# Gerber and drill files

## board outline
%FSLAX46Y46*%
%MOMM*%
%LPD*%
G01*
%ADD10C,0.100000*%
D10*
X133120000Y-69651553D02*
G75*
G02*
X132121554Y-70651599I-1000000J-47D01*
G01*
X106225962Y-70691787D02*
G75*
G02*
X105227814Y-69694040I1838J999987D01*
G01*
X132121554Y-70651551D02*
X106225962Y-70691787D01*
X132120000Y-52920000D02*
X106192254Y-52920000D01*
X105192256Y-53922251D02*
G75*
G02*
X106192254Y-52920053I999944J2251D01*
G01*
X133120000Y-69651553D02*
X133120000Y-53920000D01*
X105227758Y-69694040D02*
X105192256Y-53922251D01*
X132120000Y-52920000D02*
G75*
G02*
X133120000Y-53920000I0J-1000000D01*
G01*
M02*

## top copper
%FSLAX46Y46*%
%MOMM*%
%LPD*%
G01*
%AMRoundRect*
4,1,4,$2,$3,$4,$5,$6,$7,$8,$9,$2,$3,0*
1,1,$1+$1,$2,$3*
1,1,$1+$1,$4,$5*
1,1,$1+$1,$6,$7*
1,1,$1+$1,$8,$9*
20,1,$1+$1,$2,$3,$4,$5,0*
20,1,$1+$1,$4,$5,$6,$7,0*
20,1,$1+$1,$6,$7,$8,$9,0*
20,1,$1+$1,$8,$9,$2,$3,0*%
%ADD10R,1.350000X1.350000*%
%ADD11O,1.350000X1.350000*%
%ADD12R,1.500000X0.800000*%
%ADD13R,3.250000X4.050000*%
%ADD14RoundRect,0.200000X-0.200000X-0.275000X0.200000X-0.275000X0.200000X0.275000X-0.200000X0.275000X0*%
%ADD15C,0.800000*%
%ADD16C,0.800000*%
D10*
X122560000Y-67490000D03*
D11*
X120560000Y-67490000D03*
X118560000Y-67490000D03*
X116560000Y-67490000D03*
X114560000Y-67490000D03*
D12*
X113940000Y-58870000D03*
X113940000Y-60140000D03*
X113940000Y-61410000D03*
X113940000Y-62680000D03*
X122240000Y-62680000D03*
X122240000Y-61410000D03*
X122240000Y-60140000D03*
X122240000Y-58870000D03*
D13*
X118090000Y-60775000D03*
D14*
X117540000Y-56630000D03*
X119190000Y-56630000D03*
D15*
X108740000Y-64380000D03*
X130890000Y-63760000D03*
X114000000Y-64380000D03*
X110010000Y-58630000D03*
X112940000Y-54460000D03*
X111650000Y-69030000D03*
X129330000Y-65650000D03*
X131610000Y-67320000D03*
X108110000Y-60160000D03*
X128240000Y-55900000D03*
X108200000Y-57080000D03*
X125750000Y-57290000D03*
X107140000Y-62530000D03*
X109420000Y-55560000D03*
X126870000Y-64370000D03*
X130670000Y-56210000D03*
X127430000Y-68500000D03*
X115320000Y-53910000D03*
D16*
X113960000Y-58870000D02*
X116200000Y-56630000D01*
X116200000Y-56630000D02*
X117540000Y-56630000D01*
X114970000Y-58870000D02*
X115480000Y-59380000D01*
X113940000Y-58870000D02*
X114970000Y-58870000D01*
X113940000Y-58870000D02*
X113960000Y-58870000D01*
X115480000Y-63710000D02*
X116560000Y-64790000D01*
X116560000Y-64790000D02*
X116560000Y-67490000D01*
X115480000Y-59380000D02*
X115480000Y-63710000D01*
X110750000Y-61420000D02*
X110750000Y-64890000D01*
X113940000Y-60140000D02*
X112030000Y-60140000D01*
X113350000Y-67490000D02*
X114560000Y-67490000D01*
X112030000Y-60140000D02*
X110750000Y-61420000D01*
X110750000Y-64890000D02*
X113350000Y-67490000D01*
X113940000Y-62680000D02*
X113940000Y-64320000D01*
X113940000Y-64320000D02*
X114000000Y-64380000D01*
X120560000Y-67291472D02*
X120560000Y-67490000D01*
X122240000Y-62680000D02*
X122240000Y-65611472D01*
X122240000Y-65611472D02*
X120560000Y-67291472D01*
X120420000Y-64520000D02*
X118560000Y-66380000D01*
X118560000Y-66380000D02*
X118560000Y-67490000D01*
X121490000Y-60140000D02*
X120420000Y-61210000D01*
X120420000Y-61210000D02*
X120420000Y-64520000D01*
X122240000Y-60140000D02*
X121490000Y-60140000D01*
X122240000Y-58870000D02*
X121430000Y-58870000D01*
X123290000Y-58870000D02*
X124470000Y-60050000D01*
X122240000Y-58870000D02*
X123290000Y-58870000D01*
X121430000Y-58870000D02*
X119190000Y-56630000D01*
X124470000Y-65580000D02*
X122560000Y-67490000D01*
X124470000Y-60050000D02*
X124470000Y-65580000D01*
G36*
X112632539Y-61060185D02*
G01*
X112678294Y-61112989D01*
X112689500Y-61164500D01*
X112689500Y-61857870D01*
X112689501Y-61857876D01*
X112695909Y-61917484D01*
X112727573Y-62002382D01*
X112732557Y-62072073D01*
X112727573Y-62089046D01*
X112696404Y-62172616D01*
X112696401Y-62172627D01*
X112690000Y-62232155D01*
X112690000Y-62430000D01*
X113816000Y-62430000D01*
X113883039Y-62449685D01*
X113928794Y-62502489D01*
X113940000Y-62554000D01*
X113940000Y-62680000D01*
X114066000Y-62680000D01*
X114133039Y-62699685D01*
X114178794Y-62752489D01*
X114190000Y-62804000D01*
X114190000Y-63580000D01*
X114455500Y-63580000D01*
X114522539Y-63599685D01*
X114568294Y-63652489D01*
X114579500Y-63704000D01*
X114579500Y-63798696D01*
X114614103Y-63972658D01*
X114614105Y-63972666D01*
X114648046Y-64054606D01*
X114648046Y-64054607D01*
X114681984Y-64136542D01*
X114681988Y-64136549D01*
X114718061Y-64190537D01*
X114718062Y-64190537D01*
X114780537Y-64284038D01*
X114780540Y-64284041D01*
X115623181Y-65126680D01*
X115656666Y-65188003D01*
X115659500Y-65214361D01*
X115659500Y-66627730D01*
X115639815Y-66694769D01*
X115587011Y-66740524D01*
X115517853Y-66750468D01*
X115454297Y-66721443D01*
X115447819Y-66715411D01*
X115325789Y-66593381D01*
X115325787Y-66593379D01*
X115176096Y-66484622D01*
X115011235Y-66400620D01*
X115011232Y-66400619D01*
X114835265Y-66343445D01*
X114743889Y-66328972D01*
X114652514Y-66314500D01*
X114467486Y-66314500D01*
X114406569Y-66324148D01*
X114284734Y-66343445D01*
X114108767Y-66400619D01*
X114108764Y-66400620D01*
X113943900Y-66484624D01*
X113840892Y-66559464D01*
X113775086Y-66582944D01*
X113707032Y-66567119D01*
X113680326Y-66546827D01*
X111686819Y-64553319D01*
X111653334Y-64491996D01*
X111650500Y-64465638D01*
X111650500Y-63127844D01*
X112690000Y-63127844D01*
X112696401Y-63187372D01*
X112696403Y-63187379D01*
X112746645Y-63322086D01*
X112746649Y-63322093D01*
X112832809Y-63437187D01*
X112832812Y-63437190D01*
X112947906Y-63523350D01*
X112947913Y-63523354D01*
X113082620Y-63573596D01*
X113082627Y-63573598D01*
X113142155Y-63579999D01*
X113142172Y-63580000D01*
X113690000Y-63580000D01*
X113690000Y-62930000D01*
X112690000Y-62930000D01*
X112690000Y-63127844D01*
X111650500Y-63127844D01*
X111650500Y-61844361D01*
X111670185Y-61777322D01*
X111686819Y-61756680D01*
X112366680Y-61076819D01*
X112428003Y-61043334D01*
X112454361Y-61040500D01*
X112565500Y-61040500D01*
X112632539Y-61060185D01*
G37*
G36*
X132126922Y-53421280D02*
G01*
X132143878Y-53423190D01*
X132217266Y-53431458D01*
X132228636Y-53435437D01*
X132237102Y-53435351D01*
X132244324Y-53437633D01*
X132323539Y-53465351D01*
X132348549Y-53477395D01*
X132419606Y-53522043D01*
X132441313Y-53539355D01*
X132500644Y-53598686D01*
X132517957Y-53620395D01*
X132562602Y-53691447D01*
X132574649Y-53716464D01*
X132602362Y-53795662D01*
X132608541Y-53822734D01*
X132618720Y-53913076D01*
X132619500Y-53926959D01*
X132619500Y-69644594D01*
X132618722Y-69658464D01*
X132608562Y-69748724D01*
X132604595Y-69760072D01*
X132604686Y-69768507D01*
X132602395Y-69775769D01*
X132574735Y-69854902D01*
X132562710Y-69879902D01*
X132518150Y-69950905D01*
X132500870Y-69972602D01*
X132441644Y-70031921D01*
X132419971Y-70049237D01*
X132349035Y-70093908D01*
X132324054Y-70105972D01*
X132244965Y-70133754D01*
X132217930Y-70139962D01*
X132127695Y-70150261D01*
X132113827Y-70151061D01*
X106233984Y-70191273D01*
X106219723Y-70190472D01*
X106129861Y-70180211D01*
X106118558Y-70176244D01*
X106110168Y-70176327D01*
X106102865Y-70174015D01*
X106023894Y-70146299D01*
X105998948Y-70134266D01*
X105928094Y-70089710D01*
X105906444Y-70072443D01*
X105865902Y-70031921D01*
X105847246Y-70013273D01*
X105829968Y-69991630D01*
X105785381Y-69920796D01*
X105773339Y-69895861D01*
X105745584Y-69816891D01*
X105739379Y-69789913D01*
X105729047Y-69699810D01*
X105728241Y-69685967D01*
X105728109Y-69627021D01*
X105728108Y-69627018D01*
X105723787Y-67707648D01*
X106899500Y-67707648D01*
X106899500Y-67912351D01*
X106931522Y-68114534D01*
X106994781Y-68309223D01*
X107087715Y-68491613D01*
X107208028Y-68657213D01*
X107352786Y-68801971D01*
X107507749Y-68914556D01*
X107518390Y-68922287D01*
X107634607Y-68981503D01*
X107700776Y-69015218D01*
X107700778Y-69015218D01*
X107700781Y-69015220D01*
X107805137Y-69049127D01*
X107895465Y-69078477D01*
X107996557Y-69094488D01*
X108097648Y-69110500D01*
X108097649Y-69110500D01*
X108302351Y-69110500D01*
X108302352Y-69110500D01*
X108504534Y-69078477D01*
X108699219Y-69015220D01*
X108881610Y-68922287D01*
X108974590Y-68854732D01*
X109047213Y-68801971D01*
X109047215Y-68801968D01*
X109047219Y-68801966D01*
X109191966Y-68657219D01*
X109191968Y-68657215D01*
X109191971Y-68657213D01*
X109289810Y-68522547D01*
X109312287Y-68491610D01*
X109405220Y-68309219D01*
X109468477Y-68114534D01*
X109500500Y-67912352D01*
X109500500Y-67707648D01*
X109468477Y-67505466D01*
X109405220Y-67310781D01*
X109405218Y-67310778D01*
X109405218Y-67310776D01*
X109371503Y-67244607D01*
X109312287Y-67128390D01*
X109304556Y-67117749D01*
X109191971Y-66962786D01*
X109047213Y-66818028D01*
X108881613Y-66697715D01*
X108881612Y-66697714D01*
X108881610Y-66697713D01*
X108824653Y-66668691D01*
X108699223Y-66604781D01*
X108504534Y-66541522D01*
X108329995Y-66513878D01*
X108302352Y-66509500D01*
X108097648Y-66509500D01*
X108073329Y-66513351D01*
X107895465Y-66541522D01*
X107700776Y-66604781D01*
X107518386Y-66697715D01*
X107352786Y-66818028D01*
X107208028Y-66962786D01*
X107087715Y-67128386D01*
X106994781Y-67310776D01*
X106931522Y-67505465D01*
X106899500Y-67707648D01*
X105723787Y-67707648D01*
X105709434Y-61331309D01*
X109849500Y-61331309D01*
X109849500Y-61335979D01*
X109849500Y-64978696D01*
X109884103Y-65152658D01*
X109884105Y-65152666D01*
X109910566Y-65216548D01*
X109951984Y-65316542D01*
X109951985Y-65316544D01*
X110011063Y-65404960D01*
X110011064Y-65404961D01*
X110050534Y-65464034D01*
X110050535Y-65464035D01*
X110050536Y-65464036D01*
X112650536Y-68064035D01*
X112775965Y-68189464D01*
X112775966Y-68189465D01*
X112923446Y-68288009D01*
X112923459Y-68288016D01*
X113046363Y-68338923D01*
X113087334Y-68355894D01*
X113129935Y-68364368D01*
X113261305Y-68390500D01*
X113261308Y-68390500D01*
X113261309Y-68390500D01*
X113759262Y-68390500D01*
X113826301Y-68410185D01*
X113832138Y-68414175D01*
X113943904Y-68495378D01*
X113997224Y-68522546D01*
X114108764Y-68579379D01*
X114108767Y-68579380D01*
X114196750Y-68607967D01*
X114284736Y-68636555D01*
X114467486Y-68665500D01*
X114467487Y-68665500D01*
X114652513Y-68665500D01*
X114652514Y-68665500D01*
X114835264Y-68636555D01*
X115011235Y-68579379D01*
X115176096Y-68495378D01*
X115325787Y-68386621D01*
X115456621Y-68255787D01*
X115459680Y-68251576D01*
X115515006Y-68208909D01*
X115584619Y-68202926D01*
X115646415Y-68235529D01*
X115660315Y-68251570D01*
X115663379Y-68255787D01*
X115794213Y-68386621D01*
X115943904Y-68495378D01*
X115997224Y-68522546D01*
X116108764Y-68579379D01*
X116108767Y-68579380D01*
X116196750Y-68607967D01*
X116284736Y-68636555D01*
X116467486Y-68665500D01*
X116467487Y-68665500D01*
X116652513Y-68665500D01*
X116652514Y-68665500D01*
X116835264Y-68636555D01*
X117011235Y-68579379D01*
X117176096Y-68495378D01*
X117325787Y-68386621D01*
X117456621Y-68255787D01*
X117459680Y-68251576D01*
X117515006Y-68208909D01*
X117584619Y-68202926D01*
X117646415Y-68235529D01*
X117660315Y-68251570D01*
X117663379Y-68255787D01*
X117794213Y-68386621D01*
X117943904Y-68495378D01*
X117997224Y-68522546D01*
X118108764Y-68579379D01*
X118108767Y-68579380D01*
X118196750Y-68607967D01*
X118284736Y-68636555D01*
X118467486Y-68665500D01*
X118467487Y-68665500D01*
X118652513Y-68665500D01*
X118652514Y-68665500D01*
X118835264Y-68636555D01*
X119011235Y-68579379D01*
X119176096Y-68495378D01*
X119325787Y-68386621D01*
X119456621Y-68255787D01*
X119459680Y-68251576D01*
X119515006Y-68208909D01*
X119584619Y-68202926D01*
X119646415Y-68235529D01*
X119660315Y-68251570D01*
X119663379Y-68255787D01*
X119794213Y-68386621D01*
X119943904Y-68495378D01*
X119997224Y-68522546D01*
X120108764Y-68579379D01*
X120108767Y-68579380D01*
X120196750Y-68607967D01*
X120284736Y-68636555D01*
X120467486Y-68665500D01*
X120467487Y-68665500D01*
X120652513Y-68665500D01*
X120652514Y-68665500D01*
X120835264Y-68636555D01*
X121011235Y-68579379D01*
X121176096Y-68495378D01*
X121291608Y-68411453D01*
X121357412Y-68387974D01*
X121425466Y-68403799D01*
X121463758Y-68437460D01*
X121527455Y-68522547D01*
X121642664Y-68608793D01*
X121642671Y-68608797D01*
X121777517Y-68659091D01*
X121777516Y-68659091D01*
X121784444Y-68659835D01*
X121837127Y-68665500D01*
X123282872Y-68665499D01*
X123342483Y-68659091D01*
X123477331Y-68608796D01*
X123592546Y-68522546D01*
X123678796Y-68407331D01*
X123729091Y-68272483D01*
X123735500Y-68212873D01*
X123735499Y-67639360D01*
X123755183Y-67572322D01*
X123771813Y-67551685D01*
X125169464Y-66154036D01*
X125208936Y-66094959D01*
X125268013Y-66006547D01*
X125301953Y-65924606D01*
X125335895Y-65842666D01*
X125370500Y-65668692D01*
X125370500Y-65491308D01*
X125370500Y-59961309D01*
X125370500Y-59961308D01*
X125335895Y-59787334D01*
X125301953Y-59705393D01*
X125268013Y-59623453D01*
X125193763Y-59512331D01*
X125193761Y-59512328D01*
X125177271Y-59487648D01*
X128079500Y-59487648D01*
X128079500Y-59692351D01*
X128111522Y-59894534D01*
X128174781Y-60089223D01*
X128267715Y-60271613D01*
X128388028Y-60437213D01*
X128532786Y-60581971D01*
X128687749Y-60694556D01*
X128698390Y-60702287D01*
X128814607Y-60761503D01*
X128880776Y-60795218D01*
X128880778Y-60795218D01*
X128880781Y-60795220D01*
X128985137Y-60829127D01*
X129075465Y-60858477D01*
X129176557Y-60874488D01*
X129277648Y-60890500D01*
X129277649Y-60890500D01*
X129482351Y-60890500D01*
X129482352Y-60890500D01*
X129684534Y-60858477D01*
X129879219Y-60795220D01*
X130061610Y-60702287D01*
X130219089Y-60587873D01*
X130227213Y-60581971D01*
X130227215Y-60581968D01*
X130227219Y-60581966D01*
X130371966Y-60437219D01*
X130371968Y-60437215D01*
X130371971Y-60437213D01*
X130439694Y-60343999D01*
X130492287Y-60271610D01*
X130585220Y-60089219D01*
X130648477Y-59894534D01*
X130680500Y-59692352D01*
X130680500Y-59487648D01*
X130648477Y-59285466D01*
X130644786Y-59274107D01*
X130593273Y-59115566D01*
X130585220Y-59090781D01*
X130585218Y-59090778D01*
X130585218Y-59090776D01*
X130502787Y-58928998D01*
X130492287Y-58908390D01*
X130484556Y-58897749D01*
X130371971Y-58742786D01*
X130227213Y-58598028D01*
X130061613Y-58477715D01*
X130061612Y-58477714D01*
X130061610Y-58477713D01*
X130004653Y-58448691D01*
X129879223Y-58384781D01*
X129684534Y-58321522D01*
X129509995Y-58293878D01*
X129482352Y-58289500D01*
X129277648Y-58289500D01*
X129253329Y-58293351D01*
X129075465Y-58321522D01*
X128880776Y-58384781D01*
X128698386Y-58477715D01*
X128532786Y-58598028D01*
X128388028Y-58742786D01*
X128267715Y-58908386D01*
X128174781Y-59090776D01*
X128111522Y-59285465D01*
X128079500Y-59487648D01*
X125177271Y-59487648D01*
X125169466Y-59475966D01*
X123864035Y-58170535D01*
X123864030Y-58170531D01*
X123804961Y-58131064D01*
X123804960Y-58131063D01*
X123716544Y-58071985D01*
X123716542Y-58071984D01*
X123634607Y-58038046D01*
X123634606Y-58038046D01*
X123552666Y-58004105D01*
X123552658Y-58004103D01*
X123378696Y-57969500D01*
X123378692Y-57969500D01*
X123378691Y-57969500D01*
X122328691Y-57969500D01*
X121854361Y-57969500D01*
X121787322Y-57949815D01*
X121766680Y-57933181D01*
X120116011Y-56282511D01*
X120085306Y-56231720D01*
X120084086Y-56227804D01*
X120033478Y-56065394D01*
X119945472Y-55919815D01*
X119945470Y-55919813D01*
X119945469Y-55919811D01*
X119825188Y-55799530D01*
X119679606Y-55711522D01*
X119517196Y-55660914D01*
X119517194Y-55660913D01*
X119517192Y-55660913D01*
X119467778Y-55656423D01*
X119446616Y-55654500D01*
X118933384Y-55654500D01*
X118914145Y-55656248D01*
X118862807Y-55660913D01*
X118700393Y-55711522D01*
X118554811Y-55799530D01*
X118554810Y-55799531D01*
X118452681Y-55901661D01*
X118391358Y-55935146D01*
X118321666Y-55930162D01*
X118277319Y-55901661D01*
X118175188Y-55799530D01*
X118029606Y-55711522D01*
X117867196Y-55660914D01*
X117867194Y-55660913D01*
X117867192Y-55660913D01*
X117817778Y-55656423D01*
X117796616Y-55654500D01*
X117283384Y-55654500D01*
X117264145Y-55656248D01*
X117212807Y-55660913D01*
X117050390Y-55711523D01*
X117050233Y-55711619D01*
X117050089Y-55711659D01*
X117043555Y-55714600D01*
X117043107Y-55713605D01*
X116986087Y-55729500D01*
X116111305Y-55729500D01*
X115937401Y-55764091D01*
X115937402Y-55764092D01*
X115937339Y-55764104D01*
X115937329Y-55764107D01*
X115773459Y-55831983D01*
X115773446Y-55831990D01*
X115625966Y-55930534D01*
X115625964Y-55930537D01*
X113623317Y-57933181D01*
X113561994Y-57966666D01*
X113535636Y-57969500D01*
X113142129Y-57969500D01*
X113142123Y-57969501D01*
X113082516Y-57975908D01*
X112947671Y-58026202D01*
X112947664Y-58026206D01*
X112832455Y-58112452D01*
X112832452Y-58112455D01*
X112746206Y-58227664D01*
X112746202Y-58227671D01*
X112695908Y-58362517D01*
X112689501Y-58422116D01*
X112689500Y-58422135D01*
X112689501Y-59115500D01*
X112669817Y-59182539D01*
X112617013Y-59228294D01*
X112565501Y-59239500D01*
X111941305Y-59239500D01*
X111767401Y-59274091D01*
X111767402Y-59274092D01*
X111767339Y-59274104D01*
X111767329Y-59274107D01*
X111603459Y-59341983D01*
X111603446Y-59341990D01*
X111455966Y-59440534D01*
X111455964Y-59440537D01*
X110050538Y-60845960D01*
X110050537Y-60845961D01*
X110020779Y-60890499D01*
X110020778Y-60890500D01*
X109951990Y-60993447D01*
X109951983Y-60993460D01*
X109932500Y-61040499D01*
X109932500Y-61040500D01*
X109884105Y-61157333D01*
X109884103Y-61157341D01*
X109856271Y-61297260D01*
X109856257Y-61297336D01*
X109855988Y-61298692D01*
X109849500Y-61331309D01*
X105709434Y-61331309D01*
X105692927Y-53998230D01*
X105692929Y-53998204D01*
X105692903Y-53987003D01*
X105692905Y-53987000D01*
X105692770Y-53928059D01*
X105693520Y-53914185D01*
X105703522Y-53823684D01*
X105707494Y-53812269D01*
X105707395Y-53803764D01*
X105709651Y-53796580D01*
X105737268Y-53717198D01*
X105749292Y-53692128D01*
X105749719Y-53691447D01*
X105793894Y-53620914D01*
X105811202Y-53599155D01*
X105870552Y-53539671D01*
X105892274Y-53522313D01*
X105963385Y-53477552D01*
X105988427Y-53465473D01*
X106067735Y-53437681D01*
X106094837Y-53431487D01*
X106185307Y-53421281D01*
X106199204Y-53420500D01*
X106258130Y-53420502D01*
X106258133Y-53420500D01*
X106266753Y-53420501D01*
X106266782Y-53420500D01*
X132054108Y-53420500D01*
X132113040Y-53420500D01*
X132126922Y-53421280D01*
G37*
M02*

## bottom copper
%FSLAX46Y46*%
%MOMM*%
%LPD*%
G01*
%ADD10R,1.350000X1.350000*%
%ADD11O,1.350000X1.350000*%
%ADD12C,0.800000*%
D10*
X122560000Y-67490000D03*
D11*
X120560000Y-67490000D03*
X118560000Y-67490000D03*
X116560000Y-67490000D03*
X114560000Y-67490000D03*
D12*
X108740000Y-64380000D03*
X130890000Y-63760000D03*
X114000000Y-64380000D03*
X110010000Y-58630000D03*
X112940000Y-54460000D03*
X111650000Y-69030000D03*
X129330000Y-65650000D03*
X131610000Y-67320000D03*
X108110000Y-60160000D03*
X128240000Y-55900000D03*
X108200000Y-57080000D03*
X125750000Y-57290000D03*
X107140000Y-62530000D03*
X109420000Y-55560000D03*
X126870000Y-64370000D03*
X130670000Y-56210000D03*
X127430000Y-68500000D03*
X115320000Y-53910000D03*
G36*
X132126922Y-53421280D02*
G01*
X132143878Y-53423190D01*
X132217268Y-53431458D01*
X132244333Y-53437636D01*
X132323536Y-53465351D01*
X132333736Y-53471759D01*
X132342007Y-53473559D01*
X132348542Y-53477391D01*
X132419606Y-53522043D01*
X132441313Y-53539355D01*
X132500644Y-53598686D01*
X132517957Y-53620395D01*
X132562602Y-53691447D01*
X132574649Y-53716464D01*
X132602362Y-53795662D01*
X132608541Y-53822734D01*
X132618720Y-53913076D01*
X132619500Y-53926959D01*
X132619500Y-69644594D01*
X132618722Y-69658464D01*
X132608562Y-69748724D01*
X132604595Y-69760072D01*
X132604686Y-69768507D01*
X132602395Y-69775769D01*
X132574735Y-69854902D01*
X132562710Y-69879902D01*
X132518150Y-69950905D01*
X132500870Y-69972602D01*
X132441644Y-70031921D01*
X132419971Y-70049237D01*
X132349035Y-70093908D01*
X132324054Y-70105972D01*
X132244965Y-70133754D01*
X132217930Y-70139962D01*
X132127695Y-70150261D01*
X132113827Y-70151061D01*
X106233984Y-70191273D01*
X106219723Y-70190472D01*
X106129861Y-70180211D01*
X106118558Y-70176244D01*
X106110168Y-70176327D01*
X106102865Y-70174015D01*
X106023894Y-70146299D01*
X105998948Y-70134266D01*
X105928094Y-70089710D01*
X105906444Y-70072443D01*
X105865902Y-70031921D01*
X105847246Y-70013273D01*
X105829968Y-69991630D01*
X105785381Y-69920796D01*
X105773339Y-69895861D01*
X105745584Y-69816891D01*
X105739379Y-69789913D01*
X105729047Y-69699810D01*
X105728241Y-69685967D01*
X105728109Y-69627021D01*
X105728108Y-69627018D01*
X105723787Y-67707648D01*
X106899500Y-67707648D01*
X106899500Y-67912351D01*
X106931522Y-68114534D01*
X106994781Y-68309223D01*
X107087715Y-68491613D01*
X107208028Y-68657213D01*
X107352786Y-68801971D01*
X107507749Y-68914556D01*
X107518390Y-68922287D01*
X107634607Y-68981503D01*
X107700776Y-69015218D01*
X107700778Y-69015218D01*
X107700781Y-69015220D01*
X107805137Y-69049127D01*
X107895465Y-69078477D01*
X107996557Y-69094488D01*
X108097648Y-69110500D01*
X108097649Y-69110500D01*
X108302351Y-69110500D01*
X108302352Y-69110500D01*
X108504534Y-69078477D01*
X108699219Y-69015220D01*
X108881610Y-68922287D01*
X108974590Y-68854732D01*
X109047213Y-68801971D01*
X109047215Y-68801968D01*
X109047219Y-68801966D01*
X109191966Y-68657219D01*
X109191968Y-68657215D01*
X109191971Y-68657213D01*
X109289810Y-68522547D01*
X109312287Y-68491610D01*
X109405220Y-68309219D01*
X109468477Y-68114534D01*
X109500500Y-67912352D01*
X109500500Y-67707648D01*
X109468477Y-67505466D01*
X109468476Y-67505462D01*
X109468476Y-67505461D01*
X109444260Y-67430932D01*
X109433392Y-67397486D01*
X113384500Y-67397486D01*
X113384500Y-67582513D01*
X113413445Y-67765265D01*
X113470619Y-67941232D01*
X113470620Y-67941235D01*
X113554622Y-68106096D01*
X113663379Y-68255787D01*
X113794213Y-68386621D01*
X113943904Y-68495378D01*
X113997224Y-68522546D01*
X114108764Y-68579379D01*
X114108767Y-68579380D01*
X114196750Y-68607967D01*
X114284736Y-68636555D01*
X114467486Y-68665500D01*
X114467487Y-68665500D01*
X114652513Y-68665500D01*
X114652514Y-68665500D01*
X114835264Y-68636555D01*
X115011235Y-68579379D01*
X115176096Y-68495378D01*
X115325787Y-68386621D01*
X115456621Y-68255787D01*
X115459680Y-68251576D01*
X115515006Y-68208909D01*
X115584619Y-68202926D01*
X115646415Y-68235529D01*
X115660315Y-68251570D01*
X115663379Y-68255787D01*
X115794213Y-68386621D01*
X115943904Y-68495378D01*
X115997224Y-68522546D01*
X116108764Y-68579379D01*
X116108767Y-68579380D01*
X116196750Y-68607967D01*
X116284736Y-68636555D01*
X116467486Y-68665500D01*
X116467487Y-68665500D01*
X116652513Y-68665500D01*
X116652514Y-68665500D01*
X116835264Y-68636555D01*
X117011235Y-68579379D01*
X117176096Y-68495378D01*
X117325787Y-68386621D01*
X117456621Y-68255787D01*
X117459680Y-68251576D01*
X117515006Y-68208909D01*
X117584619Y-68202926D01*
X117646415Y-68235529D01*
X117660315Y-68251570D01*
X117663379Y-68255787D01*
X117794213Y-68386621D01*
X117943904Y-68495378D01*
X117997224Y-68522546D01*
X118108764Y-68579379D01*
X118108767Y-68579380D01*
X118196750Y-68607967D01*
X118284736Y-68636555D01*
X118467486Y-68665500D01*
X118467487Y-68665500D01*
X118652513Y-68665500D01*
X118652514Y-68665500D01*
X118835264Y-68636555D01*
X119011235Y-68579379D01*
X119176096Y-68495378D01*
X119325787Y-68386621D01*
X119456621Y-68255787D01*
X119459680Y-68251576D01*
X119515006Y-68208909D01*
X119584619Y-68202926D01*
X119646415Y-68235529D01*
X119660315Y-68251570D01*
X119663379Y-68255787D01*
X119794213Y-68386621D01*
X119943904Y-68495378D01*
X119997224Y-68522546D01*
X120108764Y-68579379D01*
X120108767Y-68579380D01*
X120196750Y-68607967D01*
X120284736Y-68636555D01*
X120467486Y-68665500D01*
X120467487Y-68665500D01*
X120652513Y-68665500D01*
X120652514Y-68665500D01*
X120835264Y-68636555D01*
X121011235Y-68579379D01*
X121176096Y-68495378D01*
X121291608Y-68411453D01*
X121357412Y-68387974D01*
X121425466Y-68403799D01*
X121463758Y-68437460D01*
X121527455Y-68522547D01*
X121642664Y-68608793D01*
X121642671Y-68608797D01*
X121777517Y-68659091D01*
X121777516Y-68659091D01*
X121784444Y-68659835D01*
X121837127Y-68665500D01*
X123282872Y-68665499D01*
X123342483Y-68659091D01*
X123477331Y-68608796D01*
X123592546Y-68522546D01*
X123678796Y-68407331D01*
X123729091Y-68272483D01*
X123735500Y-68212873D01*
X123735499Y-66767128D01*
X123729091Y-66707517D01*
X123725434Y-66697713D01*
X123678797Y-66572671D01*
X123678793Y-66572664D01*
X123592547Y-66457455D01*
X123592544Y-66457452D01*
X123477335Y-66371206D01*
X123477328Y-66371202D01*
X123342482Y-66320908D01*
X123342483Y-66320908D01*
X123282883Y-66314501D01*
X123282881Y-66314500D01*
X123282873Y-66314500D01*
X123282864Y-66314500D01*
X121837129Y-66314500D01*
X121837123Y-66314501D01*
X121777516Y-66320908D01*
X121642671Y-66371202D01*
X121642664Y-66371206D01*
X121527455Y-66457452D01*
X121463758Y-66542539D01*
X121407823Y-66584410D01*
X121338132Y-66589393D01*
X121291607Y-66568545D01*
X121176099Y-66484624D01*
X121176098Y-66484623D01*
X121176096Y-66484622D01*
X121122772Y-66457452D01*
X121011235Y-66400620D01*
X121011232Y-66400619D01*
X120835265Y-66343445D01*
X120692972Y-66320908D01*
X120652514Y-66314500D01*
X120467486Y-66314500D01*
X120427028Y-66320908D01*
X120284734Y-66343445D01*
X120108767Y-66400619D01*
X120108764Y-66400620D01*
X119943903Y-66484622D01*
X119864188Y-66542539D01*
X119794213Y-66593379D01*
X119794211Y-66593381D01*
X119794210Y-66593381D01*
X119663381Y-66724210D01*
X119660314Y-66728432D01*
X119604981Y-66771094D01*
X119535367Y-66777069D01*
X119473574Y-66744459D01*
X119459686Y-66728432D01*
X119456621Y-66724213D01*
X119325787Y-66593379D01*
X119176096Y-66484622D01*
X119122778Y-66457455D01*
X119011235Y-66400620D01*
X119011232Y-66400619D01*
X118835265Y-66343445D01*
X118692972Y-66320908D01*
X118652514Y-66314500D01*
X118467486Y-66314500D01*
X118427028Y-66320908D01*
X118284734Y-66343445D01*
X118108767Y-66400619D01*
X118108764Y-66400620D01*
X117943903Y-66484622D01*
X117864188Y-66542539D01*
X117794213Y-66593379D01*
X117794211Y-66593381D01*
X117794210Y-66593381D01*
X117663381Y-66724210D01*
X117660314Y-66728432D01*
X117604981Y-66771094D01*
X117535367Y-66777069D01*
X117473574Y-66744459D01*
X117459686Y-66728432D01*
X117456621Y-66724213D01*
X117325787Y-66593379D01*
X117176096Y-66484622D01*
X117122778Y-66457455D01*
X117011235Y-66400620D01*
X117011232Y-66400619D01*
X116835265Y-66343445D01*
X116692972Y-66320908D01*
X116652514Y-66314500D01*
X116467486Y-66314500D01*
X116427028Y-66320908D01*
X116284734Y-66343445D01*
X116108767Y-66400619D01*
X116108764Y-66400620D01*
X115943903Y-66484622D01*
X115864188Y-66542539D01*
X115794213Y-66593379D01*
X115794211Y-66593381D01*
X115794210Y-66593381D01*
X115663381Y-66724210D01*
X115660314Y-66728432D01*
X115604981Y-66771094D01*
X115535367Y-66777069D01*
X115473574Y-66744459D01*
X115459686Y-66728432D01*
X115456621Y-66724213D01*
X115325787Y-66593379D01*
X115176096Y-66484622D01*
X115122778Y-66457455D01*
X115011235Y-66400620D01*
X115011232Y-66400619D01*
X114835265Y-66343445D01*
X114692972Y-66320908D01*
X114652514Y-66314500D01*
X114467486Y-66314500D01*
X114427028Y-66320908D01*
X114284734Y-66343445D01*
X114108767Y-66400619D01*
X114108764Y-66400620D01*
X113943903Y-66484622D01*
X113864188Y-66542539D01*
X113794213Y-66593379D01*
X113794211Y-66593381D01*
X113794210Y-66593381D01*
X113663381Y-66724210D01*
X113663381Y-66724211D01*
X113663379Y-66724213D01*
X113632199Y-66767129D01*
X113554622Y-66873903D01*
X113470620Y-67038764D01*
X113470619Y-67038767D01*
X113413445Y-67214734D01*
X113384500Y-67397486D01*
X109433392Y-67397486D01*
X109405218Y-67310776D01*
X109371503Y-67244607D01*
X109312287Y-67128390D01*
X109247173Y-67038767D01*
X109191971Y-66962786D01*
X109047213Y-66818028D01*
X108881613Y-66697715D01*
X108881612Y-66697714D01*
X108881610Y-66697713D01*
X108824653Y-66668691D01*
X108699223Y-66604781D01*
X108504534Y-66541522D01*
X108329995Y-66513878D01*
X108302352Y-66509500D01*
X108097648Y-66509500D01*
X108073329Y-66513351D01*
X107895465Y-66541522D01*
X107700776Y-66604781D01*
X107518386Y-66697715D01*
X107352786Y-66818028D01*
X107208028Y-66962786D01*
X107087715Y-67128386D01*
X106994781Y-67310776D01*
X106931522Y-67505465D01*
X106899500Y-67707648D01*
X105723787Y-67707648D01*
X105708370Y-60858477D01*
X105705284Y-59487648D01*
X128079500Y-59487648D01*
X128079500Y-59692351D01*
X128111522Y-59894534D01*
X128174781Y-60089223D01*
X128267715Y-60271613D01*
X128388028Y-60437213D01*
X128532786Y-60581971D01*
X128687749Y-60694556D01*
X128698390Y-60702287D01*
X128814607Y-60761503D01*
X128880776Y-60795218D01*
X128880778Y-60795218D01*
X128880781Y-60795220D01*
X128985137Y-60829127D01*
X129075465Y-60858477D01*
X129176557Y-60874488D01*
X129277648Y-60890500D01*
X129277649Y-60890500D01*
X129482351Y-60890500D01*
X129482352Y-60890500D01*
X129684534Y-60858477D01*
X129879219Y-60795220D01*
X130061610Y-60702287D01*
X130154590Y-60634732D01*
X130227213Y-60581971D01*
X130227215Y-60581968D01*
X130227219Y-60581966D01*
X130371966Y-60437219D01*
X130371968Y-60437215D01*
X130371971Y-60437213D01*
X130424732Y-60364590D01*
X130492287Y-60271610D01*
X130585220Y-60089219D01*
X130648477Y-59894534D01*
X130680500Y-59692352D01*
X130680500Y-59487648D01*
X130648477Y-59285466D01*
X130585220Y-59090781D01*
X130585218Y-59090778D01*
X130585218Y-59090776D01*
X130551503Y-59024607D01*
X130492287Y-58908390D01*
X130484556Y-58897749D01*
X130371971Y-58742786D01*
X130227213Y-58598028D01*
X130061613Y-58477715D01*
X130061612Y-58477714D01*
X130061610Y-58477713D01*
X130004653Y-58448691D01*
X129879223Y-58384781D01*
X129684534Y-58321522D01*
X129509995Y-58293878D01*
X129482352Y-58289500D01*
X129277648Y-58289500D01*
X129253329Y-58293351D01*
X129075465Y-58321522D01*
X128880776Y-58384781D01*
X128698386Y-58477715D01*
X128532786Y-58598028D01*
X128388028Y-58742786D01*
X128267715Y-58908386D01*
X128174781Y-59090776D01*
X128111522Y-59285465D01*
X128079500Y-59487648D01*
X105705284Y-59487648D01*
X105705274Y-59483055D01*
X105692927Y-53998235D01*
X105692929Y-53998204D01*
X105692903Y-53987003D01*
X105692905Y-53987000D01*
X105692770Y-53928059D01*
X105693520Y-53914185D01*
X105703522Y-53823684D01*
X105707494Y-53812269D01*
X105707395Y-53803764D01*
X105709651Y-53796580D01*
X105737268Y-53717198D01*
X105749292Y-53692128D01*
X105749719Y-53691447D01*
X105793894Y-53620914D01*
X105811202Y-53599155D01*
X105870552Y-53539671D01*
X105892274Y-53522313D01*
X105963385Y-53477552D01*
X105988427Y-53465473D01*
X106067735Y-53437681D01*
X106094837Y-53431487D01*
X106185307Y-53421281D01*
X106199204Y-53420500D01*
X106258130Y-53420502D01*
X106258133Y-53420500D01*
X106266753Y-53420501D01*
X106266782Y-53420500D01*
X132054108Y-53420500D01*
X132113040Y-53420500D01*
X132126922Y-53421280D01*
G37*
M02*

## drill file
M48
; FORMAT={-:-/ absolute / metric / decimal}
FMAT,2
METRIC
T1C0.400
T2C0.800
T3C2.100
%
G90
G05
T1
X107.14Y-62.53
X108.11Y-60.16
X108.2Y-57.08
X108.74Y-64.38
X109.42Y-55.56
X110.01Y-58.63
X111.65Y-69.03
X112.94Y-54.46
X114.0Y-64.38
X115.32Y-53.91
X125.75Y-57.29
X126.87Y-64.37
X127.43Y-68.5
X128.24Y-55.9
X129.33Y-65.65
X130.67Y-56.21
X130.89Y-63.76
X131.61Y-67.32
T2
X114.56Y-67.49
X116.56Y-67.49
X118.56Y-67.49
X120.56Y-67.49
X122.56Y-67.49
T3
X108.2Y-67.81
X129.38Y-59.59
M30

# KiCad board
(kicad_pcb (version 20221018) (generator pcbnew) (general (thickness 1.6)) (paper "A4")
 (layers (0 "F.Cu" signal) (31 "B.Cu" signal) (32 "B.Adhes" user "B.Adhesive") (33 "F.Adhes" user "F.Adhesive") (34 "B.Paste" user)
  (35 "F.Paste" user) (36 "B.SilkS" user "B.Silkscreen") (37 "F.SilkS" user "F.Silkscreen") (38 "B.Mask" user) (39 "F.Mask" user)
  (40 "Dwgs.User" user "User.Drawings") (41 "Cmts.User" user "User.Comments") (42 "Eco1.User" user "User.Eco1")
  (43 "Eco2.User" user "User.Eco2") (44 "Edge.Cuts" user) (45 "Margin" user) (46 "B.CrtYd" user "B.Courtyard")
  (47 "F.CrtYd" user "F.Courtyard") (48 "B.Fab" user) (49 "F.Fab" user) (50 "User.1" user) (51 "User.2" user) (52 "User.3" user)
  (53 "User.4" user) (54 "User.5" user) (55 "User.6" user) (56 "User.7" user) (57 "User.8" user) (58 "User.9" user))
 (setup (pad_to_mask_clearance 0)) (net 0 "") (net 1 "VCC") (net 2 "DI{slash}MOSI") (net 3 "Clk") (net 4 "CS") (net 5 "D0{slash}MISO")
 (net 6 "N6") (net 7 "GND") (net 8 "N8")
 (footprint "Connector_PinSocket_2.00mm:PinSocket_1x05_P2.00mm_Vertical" (layer "F.Cu") (at 122.56 67.49 -90)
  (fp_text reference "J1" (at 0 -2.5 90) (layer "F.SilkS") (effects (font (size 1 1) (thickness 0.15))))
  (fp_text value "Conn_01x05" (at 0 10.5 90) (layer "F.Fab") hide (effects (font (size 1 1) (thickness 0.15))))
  (pad "1" thru_hole rect (at 0 0 270) (size 1.35 1.35) (drill 0.8) (layers "*.Cu" "*.Mask") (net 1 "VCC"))
  (pad "2" thru_hole oval (at 0 2 270) (size 1.35 1.35) (drill 0.8) (layers "*.Cu" "*.Mask") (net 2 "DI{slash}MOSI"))
  (pad "3" thru_hole oval (at 0 4 270) (size 1.35 1.35) (drill 0.8) (layers "*.Cu" "*.Mask") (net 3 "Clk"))
  (pad "4" thru_hole oval (at 0 6 270) (size 1.35 1.35) (drill 0.8) (layers "*.Cu" "*.Mask") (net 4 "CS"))
  (pad "5" thru_hole oval (at 0 8 270) (size 1.35 1.35) (drill 0.8) (layers "*.Cu" "*.Mask") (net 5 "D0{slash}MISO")))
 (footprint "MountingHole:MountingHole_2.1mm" (layer "F.Cu") (at 108.2 67.81)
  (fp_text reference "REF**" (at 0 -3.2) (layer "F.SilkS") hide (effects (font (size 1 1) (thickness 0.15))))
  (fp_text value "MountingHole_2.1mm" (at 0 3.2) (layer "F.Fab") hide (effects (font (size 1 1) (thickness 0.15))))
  (pad "" np_thru_hole circle (at 0 0) (size 2.1 2.1) (drill 2.1) (layers "*.Cu" "*.Mask")))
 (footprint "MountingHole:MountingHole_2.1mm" (layer "F.Cu") (at 129.38 59.59)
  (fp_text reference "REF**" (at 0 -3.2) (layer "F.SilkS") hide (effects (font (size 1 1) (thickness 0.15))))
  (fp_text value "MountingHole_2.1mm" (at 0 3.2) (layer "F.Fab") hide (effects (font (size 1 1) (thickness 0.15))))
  (pad "" np_thru_hole circle (at 0 0) (size 2.1 2.1) (drill 2.1) (layers "F&B.Cu" "*.Mask")))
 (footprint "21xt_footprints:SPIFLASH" (layer "F.Cu") (at 118.09 60.775)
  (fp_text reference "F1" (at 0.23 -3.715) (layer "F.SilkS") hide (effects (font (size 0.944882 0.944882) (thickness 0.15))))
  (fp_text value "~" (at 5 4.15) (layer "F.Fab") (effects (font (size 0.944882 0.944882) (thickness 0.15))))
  (pad "1" smd rect (at -4.15 -1.905) (size 1.5 0.8) (layers "F.Cu" "F.Mask") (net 4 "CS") (solder_mask_margin 0.102))
  (pad "2" smd rect (at -4.15 -0.635) (size 1.5 0.8) (layers "F.Cu" "F.Mask") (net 5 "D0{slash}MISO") (solder_mask_margin 0.102))
  (pad "3" smd rect (at -4.15 0.635) (size 1.5 0.8) (layers "F.Cu" "F.Mask") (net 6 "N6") (solder_mask_margin 0.102))
  (pad "4" smd rect (at -4.15 1.905) (size 1.5 0.8) (layers "F.Cu" "F.Mask") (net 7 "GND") (solder_mask_margin 0.102))
  (pad "5" smd rect (at 4.15 1.905) (size 1.5 0.8) (layers "F.Cu" "F.Mask") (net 2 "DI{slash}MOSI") (solder_mask_margin 0.102))
  (pad "6" smd rect (at 4.15 0.635) (size 1.5 0.8) (layers "F.Cu" "F.Mask") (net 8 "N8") (solder_mask_margin 0.102))
  (pad "7" smd rect (at 4.15 -0.635) (size 1.5 0.8) (layers "F.Cu" "F.Mask") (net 3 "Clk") (solder_mask_margin 0.102))
  (pad "8" smd rect (at 4.15 -1.905) (size 1.5 0.8) (layers "F.Cu" "F.Mask") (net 1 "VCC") (solder_mask_margin 0.102))
  (pad "9" smd rect (at 0 0) (size 3.25 4.05) (layers "F.Cu" "F.Mask") (solder_mask_margin 0.102)))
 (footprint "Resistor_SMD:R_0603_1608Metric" (layer "F.Cu") (at 118.365 56.63)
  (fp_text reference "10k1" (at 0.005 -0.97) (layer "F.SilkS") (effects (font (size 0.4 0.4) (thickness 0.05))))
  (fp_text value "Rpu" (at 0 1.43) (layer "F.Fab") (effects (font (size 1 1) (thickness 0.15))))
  (pad "1" smd roundrect (at -0.825 0) (size 0.8 0.95) (layers "F.Cu" "F.Paste" "F.Mask") (roundrect_rratio 0.25) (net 4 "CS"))
  (pad "2" smd roundrect (at 0.825 0) (size 0.8 0.95) (layers "F.Cu" "F.Paste" "F.Mask") (roundrect_rratio 0.25) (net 1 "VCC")))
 (gr_arc (start 133.12 69.651553) (mid 132.827656 70.35811) (end 132.121554 70.651551) (stroke (width 0.1) (type default))
  (layer "Edge.Cuts"))
 (gr_arc (start 106.225962 70.691787) (mid 105.520811 70.399057) (end 105.227758 69.69404) (stroke (width 0.1) (type default))
  (layer "Edge.Cuts"))
 (gr_line (start 132.121554 70.651551) (end 106.225962 70.691787) (stroke (width 0.1) (type default)) (layer "Edge.Cuts"))
 (gr_line (start 132.12 52.92) (end 106.192254 52.92) (stroke (width 0.1) (type default)) (layer "Edge.Cuts"))
 (gr_arc (start 105.192256 53.922251) (mid 105.484349 53.213673) (end 106.192254 52.92) (stroke (width 0.1) (type default))
  (layer "Edge.Cuts"))
 (gr_line (start 133.12 69.651553) (end 133.12 53.92) (stroke (width 0.1) (type default)) (layer "Edge.Cuts"))
 (gr_line (start 105.227758 69.69404) (end 105.192256 53.922251) (stroke (width 0.1) (type default)) (layer "Edge.Cuts"))
 (gr_arc (start 132.12 52.92) (mid 132.827107 53.212893) (end 133.12 53.92) (stroke (width 0.1) (type default)) (layer "Edge.Cuts"))
 (segment (start 113.96 58.87) (end 116.2 56.63) (width 0.8) (layer "F.Cu") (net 4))
 (segment (start 116.2 56.63) (end 117.54 56.63) (width 0.8) (layer "F.Cu") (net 4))
 (segment (start 114.97 58.87) (end 115.48 59.38) (width 0.8) (layer "F.Cu") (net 4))
 (segment (start 113.94 58.87) (end 114.97 58.87) (width 0.8) (layer "F.Cu") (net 4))
 (segment (start 113.94 58.87) (end 113.96 58.87) (width 0.8) (layer "F.Cu") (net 4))
 (segment (start 115.48 63.71) (end 116.56 64.79) (width 0.8) (layer "F.Cu") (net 4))
 (segment (start 116.56 64.79) (end 116.56 67.49) (width 0.8) (layer "F.Cu") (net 4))
 (segment (start 115.48 59.38) (end 115.48 63.71) (width 0.8) (layer "F.Cu") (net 4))
 (segment (start 110.75 61.42) (end 110.75 64.89) (width 0.8) (layer "F.Cu") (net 5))
 (segment (start 113.94 60.14) (end 112.03 60.14) (width 0.8) (layer "F.Cu") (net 5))
 (segment (start 113.35 67.49) (end 114.56 67.49) (width 0.8) (layer "F.Cu") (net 5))
 (segment (start 112.03 60.14) (end 110.75 61.42) (width 0.8) (layer "F.Cu") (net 5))
 (segment (start 110.75 64.89) (end 113.35 67.49) (width 0.8) (layer "F.Cu") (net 5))
 (segment (start 113.94 62.68) (end 113.94 64.32) (width 0.8) (layer "F.Cu") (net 7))
 (segment (start 113.94 64.32) (end 114 64.38) (width 0.8) (layer "F.Cu") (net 7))
 (via (at 108.74 64.38) (size 0.8) (drill 0.4) (layers "F.Cu" "B.Cu") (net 7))
 (via (at 130.89 63.76) (size 0.8) (drill 0.4) (layers "F.Cu" "B.Cu") (free) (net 7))
 (via (at 114 64.38) (size 0.8) (drill 0.4) (layers "F.Cu" "B.Cu") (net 7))
 (via (at 110.01 58.63) (size 0.8) (drill 0.4) (layers "F.Cu" "B.Cu") (free) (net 7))
 (via (at 112.94 54.46) (size 0.8) (drill 0.4) (layers "F.Cu" "B.Cu") (free) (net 7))
 (via (at 111.65 69.03) (size 0.8) (drill 0.4) (layers "F.Cu" "B.Cu") (free) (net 7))
 (via (at 129.33 65.65) (size 0.8) (drill 0.4) (layers "F.Cu" "B.Cu") (free) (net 7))
 (via (at 131.61 67.32) (size 0.8) (drill 0.4) (layers "F.Cu" "B.Cu") (free) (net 7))
 (via (at 108.11 60.16) (size 0.8) (drill 0.4) (layers "F.Cu" "B.Cu") (free) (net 7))
 (via (at 128.24 55.9) (size 0.8) (drill 0.4) (layers "F.Cu" "B.Cu") (free) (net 7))
 (via (at 108.2 57.08) (size 0.8) (drill 0.4) (layers "F.Cu" "B.Cu") (free) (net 7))
 (via (at 125.75 57.29) (size 0.8) (drill 0.4) (layers "F.Cu" "B.Cu") (free) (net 7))
 (via (at 107.14 62.53) (size 0.8) (drill 0.4) (layers "F.Cu" "B.Cu") (free) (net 7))
 (via (at 109.42 55.56) (size 0.8) (drill 0.4) (layers "F.Cu" "B.Cu") (free) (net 7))
 (via (at 126.87 64.37) (size 0.8) (drill 0.4) (layers "F.Cu" "B.Cu") (free) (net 7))
 (via (at 130.67 56.21) (size 0.8) (drill 0.4) (layers "F.Cu" "B.Cu") (free) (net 7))
 (via (at 127.43 68.5) (size 0.8) (drill 0.4) (layers "F.Cu" "B.Cu") (free) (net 7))
 (via (at 115.32 53.91) (size 0.8) (drill 0.4) (layers "F.Cu" "B.Cu") (free) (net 7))
 (segment (start 120.56 67.291472) (end 120.56 67.49) (width 0.8) (layer "F.Cu") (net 2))
 (segment (start 122.24 62.68) (end 122.24 65.611472) (width 0.8) (layer "F.Cu") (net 2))
 (segment (start 122.24 65.611472) (end 120.56 67.291472) (width 0.8) (layer "F.Cu") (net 2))
 (segment (start 120.42 64.52) (end 118.56 66.38) (width 0.8) (layer "F.Cu") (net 3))
 (segment (start 118.56 66.38) (end 118.56 67.49) (width 0.8) (layer "F.Cu") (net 3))
 (segment (start 121.49 60.14) (end 120.42 61.21) (width 0.8) (layer "F.Cu") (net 3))
 (segment (start 120.42 61.21) (end 120.42 64.52) (width 0.8) (layer "F.Cu") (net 3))
 (segment (start 122.24 60.14) (end 121.49 60.14) (width 0.8) (layer "F.Cu") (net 3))
 (segment (start 122.24 58.87) (end 121.43 58.87) (width 0.8) (layer "F.Cu") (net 1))
 (segment (start 123.29 58.87) (end 124.47 60.05) (width 0.8) (layer "F.Cu") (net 1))
 (segment (start 122.24 58.87) (end 123.29 58.87) (width 0.8) (layer "F.Cu") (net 1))
 (segment (start 121.43 58.87) (end 119.19 56.63) (width 0.8) (layer "F.Cu") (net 1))
 (segment (start 124.47 65.58) (end 122.56 67.49) (width 0.8) (layer "F.Cu") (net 1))
 (segment (start 124.47 60.05) (end 124.47 65.58) (width 0.8) (layer "F.Cu") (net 1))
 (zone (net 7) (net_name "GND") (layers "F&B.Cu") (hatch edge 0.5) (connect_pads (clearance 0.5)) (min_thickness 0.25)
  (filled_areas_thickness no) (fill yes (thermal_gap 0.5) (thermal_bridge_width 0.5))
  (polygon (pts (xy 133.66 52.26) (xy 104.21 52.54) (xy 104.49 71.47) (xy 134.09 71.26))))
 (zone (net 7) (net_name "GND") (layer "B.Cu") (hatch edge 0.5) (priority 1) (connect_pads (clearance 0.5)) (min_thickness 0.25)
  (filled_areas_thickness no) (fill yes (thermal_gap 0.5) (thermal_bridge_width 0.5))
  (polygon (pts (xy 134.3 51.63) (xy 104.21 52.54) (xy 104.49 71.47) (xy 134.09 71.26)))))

